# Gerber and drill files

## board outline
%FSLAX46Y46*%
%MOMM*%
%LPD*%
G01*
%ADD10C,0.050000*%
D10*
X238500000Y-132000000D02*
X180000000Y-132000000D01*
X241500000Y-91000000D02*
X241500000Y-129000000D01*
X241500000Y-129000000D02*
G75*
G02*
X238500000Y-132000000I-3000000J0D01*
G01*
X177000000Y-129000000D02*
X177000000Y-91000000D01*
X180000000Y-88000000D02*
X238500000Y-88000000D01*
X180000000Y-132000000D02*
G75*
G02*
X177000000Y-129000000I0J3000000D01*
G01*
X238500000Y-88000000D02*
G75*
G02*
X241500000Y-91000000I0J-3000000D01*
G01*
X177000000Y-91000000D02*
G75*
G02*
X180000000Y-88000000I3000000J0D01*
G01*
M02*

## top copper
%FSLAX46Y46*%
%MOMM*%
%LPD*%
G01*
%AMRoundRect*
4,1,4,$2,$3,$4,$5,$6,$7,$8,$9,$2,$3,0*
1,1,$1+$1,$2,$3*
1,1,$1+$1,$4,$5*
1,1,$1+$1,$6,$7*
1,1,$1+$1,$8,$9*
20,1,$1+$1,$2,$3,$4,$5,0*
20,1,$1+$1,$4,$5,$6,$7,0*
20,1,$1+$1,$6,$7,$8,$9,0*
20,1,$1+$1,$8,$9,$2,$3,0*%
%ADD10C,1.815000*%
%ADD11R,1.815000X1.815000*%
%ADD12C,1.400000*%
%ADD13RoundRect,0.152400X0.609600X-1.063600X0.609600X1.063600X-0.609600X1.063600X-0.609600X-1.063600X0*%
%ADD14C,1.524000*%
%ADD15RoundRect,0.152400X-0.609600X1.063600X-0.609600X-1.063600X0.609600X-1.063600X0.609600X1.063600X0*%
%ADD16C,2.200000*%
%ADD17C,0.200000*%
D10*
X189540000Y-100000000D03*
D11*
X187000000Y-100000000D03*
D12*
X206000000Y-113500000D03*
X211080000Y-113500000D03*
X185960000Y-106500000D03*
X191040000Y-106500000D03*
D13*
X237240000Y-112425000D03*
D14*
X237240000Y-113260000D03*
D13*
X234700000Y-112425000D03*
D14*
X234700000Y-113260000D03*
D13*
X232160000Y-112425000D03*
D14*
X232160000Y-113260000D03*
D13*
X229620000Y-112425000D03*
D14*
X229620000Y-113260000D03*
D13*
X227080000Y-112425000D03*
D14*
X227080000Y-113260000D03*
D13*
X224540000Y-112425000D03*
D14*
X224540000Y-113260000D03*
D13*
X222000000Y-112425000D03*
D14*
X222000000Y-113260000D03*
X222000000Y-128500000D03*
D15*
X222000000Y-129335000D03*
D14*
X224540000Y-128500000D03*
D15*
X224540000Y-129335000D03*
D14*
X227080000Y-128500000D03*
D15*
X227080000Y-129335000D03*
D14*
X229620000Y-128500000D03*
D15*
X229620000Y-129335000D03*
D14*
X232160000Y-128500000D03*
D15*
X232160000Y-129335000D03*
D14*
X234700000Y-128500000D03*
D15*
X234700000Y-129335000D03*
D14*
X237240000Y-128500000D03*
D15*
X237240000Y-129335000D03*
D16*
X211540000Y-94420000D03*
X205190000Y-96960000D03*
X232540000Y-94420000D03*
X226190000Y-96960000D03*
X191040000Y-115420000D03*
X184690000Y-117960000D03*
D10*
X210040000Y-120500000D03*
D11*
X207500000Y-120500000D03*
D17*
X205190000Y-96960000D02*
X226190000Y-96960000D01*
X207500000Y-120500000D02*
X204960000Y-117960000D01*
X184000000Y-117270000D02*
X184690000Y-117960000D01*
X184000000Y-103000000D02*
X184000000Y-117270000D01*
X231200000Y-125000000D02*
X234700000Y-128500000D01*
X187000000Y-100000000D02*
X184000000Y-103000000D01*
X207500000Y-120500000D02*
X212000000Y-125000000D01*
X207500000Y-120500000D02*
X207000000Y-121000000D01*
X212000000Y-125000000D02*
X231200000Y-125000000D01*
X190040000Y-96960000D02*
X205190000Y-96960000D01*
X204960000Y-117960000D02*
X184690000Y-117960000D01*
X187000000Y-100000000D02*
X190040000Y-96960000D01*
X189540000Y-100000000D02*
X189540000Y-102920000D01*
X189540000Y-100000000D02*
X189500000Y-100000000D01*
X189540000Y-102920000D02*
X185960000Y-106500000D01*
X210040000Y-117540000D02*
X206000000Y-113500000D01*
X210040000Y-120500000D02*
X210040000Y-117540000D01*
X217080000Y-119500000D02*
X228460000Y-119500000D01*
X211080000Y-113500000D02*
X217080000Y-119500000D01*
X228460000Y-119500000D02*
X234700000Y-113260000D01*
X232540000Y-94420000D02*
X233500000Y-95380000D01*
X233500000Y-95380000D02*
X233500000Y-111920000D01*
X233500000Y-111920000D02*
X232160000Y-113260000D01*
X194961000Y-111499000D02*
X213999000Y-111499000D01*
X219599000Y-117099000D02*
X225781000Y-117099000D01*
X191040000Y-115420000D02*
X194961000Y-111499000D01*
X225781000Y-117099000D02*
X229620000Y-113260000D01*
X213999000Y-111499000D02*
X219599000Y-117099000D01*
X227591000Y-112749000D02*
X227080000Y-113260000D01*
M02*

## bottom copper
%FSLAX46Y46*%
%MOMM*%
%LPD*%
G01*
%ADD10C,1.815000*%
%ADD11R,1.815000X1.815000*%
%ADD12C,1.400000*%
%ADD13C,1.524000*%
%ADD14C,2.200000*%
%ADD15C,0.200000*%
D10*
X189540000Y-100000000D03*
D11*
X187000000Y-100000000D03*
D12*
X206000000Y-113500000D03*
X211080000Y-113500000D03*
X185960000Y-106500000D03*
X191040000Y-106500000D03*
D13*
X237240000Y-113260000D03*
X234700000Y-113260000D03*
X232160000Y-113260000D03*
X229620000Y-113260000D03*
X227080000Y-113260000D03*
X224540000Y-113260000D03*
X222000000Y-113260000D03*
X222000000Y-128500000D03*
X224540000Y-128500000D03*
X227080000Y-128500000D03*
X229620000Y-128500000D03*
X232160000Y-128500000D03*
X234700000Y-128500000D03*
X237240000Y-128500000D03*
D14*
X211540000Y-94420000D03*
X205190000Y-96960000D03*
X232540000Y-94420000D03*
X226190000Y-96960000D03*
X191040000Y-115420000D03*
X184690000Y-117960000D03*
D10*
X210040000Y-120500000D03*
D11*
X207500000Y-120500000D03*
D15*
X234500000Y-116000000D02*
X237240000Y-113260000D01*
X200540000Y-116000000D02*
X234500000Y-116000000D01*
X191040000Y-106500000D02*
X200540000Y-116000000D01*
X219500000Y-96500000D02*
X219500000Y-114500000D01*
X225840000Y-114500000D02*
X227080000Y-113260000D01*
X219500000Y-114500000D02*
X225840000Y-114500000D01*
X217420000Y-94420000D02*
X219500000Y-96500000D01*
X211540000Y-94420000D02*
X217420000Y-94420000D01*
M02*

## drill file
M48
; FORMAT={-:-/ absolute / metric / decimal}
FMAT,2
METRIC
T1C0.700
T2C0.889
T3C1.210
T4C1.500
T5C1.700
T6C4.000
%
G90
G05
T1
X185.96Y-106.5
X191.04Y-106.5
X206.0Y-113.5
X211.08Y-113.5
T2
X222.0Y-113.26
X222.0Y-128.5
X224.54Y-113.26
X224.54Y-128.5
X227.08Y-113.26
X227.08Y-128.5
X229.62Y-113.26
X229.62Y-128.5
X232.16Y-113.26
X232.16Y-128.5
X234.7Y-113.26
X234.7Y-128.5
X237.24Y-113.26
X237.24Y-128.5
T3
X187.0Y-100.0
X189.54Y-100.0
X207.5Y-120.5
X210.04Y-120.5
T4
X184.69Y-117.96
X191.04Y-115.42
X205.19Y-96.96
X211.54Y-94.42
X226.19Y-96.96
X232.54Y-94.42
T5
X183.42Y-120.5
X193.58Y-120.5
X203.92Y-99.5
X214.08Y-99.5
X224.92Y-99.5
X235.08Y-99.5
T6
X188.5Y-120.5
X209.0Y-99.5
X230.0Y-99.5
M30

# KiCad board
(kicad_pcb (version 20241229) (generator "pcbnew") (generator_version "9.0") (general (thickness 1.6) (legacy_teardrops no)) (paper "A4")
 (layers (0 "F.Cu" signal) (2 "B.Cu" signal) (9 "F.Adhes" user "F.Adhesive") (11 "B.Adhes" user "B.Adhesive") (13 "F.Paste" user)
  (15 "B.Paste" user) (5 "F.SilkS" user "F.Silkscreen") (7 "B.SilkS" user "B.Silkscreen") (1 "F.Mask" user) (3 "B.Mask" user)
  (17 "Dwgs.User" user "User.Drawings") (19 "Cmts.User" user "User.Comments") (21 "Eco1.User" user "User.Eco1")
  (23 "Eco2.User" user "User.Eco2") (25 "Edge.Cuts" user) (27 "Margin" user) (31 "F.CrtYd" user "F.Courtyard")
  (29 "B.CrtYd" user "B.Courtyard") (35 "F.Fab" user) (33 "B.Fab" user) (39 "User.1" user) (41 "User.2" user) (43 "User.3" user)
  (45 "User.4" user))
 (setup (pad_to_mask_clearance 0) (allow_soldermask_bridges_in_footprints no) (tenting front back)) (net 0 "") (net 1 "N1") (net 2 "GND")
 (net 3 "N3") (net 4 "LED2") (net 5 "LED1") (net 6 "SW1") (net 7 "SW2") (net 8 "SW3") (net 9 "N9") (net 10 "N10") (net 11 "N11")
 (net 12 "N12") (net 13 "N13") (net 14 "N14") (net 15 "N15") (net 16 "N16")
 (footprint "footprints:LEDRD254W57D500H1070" (layer "F.Cu") (at 188.27 100)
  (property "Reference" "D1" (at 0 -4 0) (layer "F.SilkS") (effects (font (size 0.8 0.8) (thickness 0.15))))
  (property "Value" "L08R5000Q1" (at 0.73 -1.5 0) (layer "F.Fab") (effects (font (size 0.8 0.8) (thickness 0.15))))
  (pad "A" thru_hole circle (at 1.27 0) (size 1.815 1.815) (drill 1.21) (layers "*.Cu" "*.Mask") (remove_unused_layers no) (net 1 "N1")
   (solder_mask_margin 0.102))
  (pad "C" thru_hole rect (at -1.27 0) (size 1.815 1.815) (drill 1.21) (layers "*.Cu" "*.Mask") (remove_unused_layers no) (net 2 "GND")
   (solder_mask_margin 0.102)))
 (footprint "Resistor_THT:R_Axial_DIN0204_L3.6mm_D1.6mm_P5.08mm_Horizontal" (layer "F.Cu") (at 206 113.5)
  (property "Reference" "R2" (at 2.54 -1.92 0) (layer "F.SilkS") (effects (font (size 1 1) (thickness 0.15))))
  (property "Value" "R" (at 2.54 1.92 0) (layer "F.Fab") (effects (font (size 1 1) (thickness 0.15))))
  (pad "1" thru_hole circle (at 0 0) (size 1.4 1.4) (drill 0.7) (layers "*.Cu" "*.Mask") (remove_unused_layers no) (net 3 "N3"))
  (pad "2" thru_hole circle (at 5.08 0) (size 1.4 1.4) (drill 0.7) (layers "*.Cu" "*.Mask") (remove_unused_layers no) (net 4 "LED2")))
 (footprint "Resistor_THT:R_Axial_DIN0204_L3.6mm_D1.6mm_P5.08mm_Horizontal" (layer "F.Cu") (at 185.96 106.5)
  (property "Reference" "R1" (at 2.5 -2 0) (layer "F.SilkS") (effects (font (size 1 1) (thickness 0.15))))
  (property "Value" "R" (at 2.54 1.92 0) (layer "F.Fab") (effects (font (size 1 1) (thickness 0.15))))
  (pad "1" thru_hole circle (at 0 0) (size 1.4 1.4) (drill 0.7) (layers "*.Cu" "*.Mask") (remove_unused_layers no) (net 1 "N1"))
  (pad "2" thru_hole circle (at 5.08 0) (size 1.4 1.4) (drill 0.7) (layers "*.Cu" "*.Mask") (remove_unused_layers no) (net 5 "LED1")))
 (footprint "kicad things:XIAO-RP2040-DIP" (layer "F.Cu") (at 229.62 120.88 -90)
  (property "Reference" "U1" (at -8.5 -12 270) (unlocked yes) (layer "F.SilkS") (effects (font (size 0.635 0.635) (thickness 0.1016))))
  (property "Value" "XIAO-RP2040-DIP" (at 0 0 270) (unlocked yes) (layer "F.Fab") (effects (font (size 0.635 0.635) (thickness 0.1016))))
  (pad "1" smd roundrect (at -8.455 -7.62 90) (size 2.432 1.524) (layers "F.Cu" "F.Mask") (roundrect_rratio 0.1) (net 5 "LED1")
   (thermal_bridge_angle 45))
  (pad "1" thru_hole circle (at -7.62 -7.62 90) (size 1.524 1.524) (drill 0.889) (layers "*.Cu" "*.Mask") (remove_unused_layers no)
   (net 5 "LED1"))
  (pad "2" smd roundrect (at -8.455 -5.08 90) (size 2.432 1.524) (layers "F.Cu" "F.Mask") (roundrect_rratio 0.1) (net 4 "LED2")
   (thermal_bridge_angle 45))
  (pad "2" thru_hole circle (at -7.62 -5.08 90) (size 1.524 1.524) (drill 0.889) (layers "*.Cu" "*.Mask") (remove_unused_layers no)
   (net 4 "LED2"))
  (pad "3" smd roundrect (at -8.455 -2.54 90) (size 2.432 1.524) (layers "F.Cu" "F.Mask") (roundrect_rratio 0.1) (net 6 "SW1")
   (thermal_bridge_angle 45))
  (pad "3" thru_hole circle (at -7.62 -2.54 90) (size 1.524 1.524) (drill 0.889) (layers "*.Cu" "*.Mask") (remove_unused_layers no)
   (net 6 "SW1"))
  (pad "4" smd roundrect (at -8.455 0 90) (size 2.432 1.524) (layers "F.Cu" "F.Mask") (roundrect_rratio 0.1) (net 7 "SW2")
   (thermal_bridge_angle 45))
  (pad "4" thru_hole circle (at -7.62 0 90) (size 1.524 1.524) (drill 0.889) (layers "*.Cu" "*.Mask") (remove_unused_layers no)
   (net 7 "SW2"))
  (pad "5" smd roundrect (at -8.455 2.54 90) (size 2.432 1.524) (layers "F.Cu" "F.Mask") (roundrect_rratio 0.1) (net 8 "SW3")
   (thermal_bridge_angle 45))
  (pad "5" thru_hole circle (at -7.62 2.54 90) (size 1.524 1.524) (drill 0.889) (layers "*.Cu" "*.Mask") (remove_unused_layers no)
   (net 8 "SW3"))
  (pad "6" smd roundrect (at -8.455 5.08 90) (size 2.432 1.524) (layers "F.Cu" "F.Mask") (roundrect_rratio 0.1) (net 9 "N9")
   (thermal_bridge_angle 45))
  (pad "6" thru_hole circle (at -7.62 5.08 90) (size 1.524 1.524) (drill 0.889) (layers "*.Cu" "*.Mask") (remove_unused_layers no)
   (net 9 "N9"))
  (pad "7" smd roundrect (at -8.455 7.62 90) (size 2.432 1.524) (layers "F.Cu" "F.Mask") (roundrect_rratio 0.1) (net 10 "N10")
   (thermal_bridge_angle 45))
  (pad "7" thru_hole circle (at -7.62 7.62 90) (size 1.524 1.524) (drill 0.889) (layers "*.Cu" "*.Mask") (remove_unused_layers no)
   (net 10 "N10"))
  (pad "8" thru_hole circle (at 7.62 7.62 270) (size 1.524 1.524) (drill 0.889) (layers "*.Cu" "*.Mask") (remove_unused_layers no)
   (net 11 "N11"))
  (pad "8" smd roundrect (at 8.455 7.62 270) (size 2.432 1.524) (layers "F.Cu" "F.Mask") (roundrect_rratio 0.1) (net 11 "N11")
   (thermal_bridge_angle 45))
  (pad "9" thru_hole circle (at 7.62 5.08 270) (size 1.524 1.524) (drill 0.889) (layers "*.Cu" "*.Mask") (remove_unused_layers no)
   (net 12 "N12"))
  (pad "9" smd roundrect (at 8.455 5.08 270) (size 2.432 1.524) (layers "F.Cu" "F.Mask") (roundrect_rratio 0.1) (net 12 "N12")
   (thermal_bridge_angle 45))
  (pad "10" thru_hole circle (at 7.62 2.54 270) (size 1.524 1.524) (drill 0.889) (layers "*.Cu" "*.Mask") (remove_unused_layers no)
   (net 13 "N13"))
  (pad "10" smd roundrect (at 8.455 2.54 270) (size 2.432 1.524) (layers "F.Cu" "F.Mask") (roundrect_rratio 0.1) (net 13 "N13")
   (thermal_bridge_angle 45))
  (pad "11" thru_hole circle (at 7.62 0 270) (size 1.524 1.524) (drill 0.889) (layers "*.Cu" "*.Mask") (remove_unused_layers no)
   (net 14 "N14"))
  (pad "11" smd roundrect (at 8.455 0 270) (size 2.432 1.524) (layers "F.Cu" "F.Mask") (roundrect_rratio 0.1) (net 14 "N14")
   (thermal_bridge_angle 45))
  (pad "12" thru_hole circle (at 7.62 -2.54 270) (size 1.524 1.524) (drill 0.889) (layers "*.Cu" "*.Mask") (remove_unused_layers no)
   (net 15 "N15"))
  (pad "12" smd roundrect (at 8.455 -2.54 270) (size 2.432 1.524) (layers "F.Cu" "F.Mask") (roundrect_rratio 0.1) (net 15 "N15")
   (thermal_bridge_angle 45))
  (pad "13" thru_hole circle (at 7.62 -5.08 270) (size 1.524 1.524) (drill 0.889) (layers "*.Cu" "*.Mask") (remove_unused_layers no)
   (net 2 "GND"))
  (pad "13" smd roundrect (at 8.455 -5.08 270) (size 2.432 1.524) (layers "F.Cu" "F.Mask") (roundrect_rratio 0.1) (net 2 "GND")
   (thermal_bridge_angle 45))
  (pad "14" thru_hole circle (at 7.62 -7.62 270) (size 1.524 1.524) (drill 0.889) (layers "*.Cu" "*.Mask") (remove_unused_layers no)
   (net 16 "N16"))
  (pad "14" smd roundrect (at 8.455 -7.62 270) (size 2.432 1.524) (layers "F.Cu" "F.Mask") (roundrect_rratio 0.1) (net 16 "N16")
   (thermal_bridge_angle 45)))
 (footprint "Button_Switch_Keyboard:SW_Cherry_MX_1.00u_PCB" (layer "F.Cu") (at 211.54 94.42)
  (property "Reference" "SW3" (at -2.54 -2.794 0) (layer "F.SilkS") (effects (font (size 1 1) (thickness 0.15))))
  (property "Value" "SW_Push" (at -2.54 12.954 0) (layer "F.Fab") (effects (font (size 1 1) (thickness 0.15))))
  (pad "" np_thru_hole circle (at -7.62 5.08) (size 1.7 1.7) (drill 1.7) (layers "*.Cu" "*.Mask"))
  (pad "" np_thru_hole circle (at -2.54 5.08) (size 4 4) (drill 4) (layers "*.Cu" "*.Mask"))
  (pad "" np_thru_hole circle (at 2.54 5.08) (size 1.7 1.7) (drill 1.7) (layers "*.Cu" "*.Mask"))
  (pad "1" thru_hole circle (at 0 0) (size 2.2 2.2) (drill 1.5) (layers "*.Cu" "*.Mask") (remove_unused_layers no) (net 8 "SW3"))
  (pad "2" thru_hole circle (at -6.35 2.54) (size 2.2 2.2) (drill 1.5) (layers "*.Cu" "*.Mask") (remove_unused_layers no) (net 2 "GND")))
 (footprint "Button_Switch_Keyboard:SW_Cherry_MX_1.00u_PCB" (layer "F.Cu") (at 232.54 94.42)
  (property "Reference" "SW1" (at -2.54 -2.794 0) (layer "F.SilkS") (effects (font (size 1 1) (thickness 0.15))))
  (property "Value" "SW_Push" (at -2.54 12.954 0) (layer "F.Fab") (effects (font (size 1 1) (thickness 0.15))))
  (pad "" np_thru_hole circle (at -7.62 5.08) (size 1.7 1.7) (drill 1.7) (layers "*.Cu" "*.Mask"))
  (pad "" np_thru_hole circle (at -2.54 5.08) (size 4 4) (drill 4) (layers "*.Cu" "*.Mask"))
  (pad "" np_thru_hole circle (at 2.54 5.08) (size 1.7 1.7) (drill 1.7) (layers "*.Cu" "*.Mask"))
  (pad "1" thru_hole circle (at 0 0) (size 2.2 2.2) (drill 1.5) (layers "*.Cu" "*.Mask") (remove_unused_layers no) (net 6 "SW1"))
  (pad "2" thru_hole circle (at -6.35 2.54) (size 2.2 2.2) (drill 1.5) (layers "*.Cu" "*.Mask") (remove_unused_layers no) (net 2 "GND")))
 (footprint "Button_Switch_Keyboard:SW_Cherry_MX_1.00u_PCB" (layer "F.Cu") (at 191.04 115.42)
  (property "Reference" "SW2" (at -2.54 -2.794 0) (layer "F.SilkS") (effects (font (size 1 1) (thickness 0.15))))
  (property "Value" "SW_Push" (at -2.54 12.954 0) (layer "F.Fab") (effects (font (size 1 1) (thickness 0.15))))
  (pad "" np_thru_hole circle (at -7.62 5.08) (size 1.7 1.7) (drill 1.7) (layers "*.Cu" "*.Mask"))
  (pad "" np_thru_hole circle (at -2.54 5.08) (size 4 4) (drill 4) (layers "*.Cu" "*.Mask"))
  (pad "" np_thru_hole circle (at 2.54 5.08) (size 1.7 1.7) (drill 1.7) (layers "*.Cu" "*.Mask"))
  (pad "1" thru_hole circle (at 0 0) (size 2.2 2.2) (drill 1.5) (layers "*.Cu" "*.Mask") (remove_unused_layers no) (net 7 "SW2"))
  (pad "2" thru_hole circle (at -6.35 2.54) (size 2.2 2.2) (drill 1.5) (layers "*.Cu" "*.Mask") (remove_unused_layers no) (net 2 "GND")))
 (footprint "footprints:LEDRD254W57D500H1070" (layer "F.Cu") (at 208.77 120.5)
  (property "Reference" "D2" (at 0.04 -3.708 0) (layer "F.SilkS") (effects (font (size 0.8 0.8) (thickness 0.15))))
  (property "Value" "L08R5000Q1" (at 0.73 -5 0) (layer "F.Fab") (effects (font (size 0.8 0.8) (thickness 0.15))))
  (pad "A" thru_hole circle (at 1.27 0) (size 1.815 1.815) (drill 1.21) (layers "*.Cu" "*.Mask") (remove_unused_layers no) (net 3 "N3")
   (solder_mask_margin 0.102))
  (pad "C" thru_hole rect (at -1.27 0) (size 1.815 1.815) (drill 1.21) (layers "*.Cu" "*.Mask") (remove_unused_layers no) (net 2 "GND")
   (solder_mask_margin 0.102)))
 (gr_line (start 238.5 132) (end 180 132) (stroke (width 0.05) (type default)) (layer "Edge.Cuts"))
 (gr_line (start 241.5 91) (end 241.5 129) (stroke (width 0.05) (type default)) (layer "Edge.Cuts"))
 (gr_arc (start 241.5 129) (mid 240.62132 131.12132) (end 238.5 132) (stroke (width 0.05) (type default)) (layer "Edge.Cuts"))
 (gr_line (start 177 129) (end 177 91) (stroke (width 0.05) (type default)) (layer "Edge.Cuts"))
 (gr_line (start 180 88) (end 238.5 88) (stroke (width 0.05) (type default)) (layer "Edge.Cuts"))
 (gr_arc (start 180 132) (mid 177.87868 131.12132) (end 177 129) (stroke (width 0.05) (type default)) (layer "Edge.Cuts"))
 (gr_arc (start 238.5 88) (mid 240.62132 88.87868) (end 241.5 91) (stroke (width 0.05) (type default)) (layer "Edge.Cuts"))
 (gr_arc (start 177 91) (mid 177.87868 88.87868) (end 180 88) (stroke (width 0.05) (type default)) (layer "Edge.Cuts"))
 (segment (start 205.19 96.96) (end 226.19 96.96) (width 0.2) (layer "F.Cu") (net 2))
 (segment (start 207.5 120.5) (end 204.96 117.96) (width 0.2) (layer "F.Cu") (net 2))
 (segment (start 184 117.27) (end 184.69 117.96) (width 0.2) (layer "F.Cu") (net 2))
 (segment (start 184 103) (end 184 117.27) (width 0.2) (layer "F.Cu") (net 2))
 (segment (start 231.2 125) (end 234.7 128.5) (width 0.2) (layer "F.Cu") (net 2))
 (segment (start 187 100) (end 184 103) (width 0.2) (layer "F.Cu") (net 2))
 (segment (start 207.5 120.5) (end 212 125) (width 0.2) (layer "F.Cu") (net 2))
 (segment (start 207.5 120.5) (end 207 121) (width 0.2) (layer "F.Cu") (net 2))
 (segment (start 212 125) (end 231.2 125) (width 0.2) (layer "F.Cu") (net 2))
 (segment (start 190.04 96.96) (end 205.19 96.96) (width 0.2) (layer "F.Cu") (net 2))
 (segment (start 204.96 117.96) (end 184.69 117.96) (width 0.2) (layer "F.Cu") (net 2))
 (segment (start 187 100) (end 190.04 96.96) (width 0.2) (layer "F.Cu") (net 2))
 (segment (start 189.54 100) (end 189.54 102.92) (width 0.2) (layer "F.Cu") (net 1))
 (segment (start 189.54 100) (end 189.5 100) (width 0.2) (layer "F.Cu") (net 1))
 (segment (start 189.54 102.92) (end 185.96 106.5) (width 0.2) (layer "F.Cu") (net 1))
 (segment (start 210.04 117.54) (end 206 113.5) (width 0.2) (layer "F.Cu") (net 3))
 (segment (start 210.04 120.5) (end 210.04 117.54) (width 0.2) (layer "F.Cu") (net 3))
 (segment (start 234.5 116) (end 237.24 113.26) (width 0.2) (layer "B.Cu") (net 5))
 (segment (start 200.54 116) (end 234.5 116) (width 0.2) (layer "B.Cu") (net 5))
 (segment (start 191.04 106.5) (end 200.54 116) (width 0.2) (layer "B.Cu") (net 5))
 (segment (start 217.08 119.5) (end 228.46 119.5) (width 0.2) (layer "F.Cu") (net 4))
 (segment (start 211.08 113.5) (end 217.08 119.5) (width 0.2) (layer "F.Cu") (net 4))
 (segment (start 228.46 119.5) (end 234.7 113.26) (width 0.2) (layer "F.Cu") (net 4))
 (segment (start 232.54 94.42) (end 233.5 95.38) (width 0.2) (layer "F.Cu") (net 6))
 (segment (start 233.5 95.38) (end 233.5 111.92) (width 0.2) (layer "F.Cu") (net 6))
 (segment (start 233.5 111.92) (end 232.16 113.26) (width 0.2) (layer "F.Cu") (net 6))
 (segment (start 194.961 111.499) (end 213.999 111.499) (width 0.2) (layer "F.Cu") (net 7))
 (segment (start 219.599 117.099) (end 225.781 117.099) (width 0.2) (layer "F.Cu") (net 7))
 (segment (start 191.04 115.42) (end 194.961 111.499) (width 0.2) (layer "F.Cu") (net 7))
 (segment (start 225.781 117.099) (end 229.62 113.26) (width 0.2) (layer "F.Cu") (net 7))
 (segment (start 213.999 111.499) (end 219.599 117.099) (width 0.2) (layer "F.Cu") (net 7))
 (segment (start 227.591 112.749) (end 227.08 113.26) (width 0.2) (layer "F.Cu") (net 8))
 (segment (start 219.5 96.5) (end 219.5 114.5) (width 0.2) (layer "B.Cu") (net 8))
 (segment (start 225.84 114.5) (end 227.08 113.26) (width 0.2) (layer "B.Cu") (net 8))
 (segment (start 219.5 114.5) (end 225.84 114.5) (width 0.2) (layer "B.Cu") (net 8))
 (segment (start 217.42 94.42) (end 219.5 96.5) (width 0.2) (layer "B.Cu") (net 8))
 (segment (start 211.54 94.42) (end 217.42 94.42) (width 0.2) (layer "B.Cu") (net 8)))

